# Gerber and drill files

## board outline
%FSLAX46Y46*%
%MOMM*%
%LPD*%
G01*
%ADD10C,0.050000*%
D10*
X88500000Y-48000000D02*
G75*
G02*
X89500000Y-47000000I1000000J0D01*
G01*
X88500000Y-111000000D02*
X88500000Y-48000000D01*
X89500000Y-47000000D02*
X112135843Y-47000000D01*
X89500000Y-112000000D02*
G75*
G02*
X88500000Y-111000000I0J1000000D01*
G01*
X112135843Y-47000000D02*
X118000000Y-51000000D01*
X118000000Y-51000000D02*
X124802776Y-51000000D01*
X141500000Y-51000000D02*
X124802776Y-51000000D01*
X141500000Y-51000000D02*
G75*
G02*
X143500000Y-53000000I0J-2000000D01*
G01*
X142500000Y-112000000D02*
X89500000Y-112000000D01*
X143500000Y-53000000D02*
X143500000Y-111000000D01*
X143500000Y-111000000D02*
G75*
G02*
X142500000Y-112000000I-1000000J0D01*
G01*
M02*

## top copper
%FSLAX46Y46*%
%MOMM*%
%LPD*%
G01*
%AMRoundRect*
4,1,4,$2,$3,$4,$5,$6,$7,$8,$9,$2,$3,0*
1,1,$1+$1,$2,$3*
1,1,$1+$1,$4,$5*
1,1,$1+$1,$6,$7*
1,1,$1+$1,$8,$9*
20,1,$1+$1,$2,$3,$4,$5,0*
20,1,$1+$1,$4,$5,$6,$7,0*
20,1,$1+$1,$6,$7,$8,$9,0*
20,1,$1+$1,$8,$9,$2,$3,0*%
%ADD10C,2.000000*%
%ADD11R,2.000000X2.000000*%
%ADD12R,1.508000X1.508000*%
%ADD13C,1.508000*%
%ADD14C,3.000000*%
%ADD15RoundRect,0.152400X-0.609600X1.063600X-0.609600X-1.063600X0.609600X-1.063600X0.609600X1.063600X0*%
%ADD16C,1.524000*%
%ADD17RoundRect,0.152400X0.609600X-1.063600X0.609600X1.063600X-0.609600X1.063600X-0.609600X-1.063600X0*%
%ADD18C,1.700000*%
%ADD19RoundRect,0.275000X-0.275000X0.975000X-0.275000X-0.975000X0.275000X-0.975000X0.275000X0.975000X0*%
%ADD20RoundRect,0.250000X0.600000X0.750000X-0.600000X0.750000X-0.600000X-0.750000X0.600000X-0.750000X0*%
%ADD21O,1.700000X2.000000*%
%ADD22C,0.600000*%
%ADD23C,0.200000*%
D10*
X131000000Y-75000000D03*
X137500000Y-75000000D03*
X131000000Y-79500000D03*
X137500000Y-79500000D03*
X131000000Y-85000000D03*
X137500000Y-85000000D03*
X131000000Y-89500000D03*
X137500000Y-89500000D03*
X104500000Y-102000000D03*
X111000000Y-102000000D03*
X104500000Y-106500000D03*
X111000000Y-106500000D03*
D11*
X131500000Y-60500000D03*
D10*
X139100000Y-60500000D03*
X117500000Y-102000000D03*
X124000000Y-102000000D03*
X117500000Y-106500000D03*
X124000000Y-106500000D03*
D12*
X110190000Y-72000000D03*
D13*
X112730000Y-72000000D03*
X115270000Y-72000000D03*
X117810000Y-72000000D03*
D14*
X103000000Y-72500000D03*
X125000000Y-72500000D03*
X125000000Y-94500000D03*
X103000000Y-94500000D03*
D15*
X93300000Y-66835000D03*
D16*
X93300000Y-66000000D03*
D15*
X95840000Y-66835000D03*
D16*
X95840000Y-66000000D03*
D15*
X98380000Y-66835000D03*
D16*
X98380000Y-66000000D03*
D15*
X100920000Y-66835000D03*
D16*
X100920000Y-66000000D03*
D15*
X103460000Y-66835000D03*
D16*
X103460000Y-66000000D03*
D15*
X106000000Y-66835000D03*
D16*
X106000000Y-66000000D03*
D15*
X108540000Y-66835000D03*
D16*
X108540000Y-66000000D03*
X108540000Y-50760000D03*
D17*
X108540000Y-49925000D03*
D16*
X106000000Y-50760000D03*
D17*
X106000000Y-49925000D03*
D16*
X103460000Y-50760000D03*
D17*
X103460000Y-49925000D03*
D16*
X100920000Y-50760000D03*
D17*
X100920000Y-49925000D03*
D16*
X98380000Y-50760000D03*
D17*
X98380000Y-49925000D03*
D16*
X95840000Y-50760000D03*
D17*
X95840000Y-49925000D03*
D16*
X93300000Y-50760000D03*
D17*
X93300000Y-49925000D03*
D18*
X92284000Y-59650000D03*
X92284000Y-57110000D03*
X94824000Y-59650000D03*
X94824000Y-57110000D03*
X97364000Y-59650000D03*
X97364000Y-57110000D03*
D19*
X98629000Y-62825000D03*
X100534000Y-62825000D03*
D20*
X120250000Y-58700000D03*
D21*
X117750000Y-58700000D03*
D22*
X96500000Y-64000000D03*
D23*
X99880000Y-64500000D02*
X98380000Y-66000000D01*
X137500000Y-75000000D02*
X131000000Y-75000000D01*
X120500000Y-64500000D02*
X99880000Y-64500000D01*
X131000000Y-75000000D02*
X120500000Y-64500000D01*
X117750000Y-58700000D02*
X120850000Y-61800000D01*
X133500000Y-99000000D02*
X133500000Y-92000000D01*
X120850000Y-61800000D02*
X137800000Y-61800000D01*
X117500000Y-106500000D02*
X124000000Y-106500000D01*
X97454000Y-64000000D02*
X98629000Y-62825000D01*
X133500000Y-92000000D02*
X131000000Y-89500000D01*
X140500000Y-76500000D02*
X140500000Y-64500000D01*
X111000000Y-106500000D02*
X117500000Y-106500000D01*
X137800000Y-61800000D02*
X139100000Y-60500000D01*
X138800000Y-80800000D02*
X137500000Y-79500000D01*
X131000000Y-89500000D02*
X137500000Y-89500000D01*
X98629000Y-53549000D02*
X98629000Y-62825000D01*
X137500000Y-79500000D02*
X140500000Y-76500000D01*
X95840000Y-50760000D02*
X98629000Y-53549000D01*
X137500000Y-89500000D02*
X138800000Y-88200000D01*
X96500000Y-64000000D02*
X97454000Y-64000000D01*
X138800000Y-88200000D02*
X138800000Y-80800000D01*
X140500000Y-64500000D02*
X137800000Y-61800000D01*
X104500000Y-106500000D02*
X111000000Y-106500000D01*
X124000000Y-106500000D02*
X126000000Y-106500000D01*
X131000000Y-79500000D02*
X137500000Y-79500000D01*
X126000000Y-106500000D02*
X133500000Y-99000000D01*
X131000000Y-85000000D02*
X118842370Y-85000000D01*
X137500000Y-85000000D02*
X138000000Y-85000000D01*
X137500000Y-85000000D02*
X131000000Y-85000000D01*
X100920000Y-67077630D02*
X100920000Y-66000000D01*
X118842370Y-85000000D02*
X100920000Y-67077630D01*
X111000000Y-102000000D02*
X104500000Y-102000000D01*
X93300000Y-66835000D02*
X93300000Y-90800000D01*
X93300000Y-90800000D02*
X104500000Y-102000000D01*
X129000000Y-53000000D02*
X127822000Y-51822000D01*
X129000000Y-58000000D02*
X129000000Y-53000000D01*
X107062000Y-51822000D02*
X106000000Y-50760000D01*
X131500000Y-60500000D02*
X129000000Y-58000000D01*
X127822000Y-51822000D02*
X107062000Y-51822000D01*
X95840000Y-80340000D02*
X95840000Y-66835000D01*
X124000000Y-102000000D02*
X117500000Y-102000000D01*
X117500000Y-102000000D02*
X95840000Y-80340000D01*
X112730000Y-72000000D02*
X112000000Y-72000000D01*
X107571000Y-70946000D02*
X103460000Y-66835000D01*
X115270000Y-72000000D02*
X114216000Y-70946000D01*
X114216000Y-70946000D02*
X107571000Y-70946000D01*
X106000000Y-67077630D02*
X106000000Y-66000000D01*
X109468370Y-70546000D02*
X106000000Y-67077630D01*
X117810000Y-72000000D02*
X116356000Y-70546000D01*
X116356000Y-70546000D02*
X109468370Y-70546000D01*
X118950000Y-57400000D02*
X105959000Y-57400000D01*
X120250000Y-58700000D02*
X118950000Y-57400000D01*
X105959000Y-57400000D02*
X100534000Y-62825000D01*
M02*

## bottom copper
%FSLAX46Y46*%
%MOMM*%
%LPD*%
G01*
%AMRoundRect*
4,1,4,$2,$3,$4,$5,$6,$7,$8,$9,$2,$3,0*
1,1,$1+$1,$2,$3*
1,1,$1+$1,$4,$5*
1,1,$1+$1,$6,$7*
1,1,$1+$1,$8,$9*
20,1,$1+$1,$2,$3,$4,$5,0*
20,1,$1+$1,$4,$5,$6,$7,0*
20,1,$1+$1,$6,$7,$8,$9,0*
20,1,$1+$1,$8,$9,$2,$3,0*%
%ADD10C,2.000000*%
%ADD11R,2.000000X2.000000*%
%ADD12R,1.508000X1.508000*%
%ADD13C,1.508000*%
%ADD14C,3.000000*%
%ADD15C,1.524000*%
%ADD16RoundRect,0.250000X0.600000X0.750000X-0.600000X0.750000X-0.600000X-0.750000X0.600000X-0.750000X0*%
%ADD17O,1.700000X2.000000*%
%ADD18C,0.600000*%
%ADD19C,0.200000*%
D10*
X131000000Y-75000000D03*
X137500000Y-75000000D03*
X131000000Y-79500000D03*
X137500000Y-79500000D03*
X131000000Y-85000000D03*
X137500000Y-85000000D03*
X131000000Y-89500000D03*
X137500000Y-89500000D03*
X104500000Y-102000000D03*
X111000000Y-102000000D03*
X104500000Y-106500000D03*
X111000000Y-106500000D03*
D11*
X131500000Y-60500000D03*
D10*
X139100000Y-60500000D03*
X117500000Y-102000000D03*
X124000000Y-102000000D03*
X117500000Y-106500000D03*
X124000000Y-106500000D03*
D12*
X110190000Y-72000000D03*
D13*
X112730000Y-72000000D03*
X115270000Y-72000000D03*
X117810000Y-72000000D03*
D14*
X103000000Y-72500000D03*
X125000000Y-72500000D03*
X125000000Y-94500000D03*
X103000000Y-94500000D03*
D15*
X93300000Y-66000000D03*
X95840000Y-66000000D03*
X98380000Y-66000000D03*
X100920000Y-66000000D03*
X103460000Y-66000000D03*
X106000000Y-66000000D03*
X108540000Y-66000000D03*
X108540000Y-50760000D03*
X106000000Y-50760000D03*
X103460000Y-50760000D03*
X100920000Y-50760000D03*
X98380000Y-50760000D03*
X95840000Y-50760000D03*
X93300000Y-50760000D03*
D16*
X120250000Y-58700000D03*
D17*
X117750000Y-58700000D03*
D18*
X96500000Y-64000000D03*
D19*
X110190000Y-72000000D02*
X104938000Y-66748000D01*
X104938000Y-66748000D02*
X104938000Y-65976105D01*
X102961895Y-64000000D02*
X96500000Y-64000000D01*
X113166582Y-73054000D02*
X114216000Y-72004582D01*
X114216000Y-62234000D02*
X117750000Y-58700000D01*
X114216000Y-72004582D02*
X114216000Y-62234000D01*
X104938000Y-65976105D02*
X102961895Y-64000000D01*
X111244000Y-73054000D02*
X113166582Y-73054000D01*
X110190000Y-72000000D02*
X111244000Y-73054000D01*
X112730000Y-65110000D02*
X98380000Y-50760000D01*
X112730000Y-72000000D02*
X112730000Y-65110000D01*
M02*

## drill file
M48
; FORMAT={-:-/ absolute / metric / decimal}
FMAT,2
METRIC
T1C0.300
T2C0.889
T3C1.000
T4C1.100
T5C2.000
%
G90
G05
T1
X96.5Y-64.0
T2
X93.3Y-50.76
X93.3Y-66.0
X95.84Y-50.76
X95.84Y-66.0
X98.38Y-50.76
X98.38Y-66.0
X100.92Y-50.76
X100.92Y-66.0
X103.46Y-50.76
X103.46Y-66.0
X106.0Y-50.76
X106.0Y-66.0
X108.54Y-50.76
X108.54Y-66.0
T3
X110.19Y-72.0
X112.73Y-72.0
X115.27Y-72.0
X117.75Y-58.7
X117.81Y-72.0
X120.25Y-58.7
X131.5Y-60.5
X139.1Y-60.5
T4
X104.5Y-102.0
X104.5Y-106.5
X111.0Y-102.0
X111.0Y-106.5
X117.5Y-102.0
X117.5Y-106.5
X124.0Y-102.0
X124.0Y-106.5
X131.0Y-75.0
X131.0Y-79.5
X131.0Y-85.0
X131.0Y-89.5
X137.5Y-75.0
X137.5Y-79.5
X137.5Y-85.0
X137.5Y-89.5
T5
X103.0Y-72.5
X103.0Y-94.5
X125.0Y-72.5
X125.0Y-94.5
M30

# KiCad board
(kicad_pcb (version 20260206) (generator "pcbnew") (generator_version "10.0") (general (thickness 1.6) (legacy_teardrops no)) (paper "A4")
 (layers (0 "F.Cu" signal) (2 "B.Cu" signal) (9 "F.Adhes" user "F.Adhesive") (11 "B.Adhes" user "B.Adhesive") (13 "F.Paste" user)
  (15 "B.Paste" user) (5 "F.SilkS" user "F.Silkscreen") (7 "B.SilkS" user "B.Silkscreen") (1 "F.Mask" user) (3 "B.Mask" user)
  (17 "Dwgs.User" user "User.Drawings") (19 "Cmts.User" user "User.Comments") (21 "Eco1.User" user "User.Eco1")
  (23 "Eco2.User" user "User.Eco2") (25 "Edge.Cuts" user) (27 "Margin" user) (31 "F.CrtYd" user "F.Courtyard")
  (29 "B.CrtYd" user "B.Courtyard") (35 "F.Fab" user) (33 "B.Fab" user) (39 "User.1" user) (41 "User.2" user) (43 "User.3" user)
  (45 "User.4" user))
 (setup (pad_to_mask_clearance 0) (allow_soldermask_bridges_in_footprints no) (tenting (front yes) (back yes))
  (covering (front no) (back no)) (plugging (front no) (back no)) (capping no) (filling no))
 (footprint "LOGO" (layer "F.Cu") (at 95 102)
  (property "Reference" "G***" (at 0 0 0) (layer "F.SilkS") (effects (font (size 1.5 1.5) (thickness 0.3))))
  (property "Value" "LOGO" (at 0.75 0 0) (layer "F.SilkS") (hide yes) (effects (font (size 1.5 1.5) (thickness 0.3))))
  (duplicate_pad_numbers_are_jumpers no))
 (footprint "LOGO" (layer "F.Cu") (at 124.5 55.5)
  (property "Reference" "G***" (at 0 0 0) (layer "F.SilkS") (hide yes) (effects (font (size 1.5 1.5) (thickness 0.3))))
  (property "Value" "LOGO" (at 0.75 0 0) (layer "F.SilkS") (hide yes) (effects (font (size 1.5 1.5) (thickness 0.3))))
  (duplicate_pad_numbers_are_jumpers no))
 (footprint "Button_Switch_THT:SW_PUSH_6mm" (layer "F.Cu") (at 131 75)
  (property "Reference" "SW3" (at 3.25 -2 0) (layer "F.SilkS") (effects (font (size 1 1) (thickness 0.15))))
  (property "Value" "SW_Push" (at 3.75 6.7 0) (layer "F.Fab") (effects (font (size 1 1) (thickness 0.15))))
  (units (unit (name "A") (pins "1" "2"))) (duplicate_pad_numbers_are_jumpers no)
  (pad "1" thru_hole circle (at 0 0 90) (size 2 2) (drill 1.1) (layers "*.Cu" "*.Mask") (remove_unused_layers no) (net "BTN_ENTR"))
  (pad "1" thru_hole circle (at 6.5 0 90) (size 2 2) (drill 1.1) (layers "*.Cu" "*.Mask") (remove_unused_layers no) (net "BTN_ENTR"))
  (pad "2" thru_hole circle (at 0 4.5 90) (size 2 2) (drill 1.1) (layers "*.Cu" "*.Mask") (remove_unused_layers no) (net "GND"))
  (pad "2" thru_hole circle (at 6.5 4.5 90) (size 2 2) (drill 1.1) (layers "*.Cu" "*.Mask") (remove_unused_layers no) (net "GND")))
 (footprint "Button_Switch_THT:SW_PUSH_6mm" (layer "F.Cu") (at 131 85)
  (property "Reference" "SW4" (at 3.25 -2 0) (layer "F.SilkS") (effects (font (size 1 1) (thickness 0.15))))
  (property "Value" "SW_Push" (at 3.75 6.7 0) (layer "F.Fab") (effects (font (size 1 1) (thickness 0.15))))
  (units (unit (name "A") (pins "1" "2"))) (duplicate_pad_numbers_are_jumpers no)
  (pad "1" thru_hole circle (at 0 0 90) (size 2 2) (drill 1.1) (layers "*.Cu" "*.Mask") (remove_unused_layers no) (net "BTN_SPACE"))
  (pad "1" thru_hole circle (at 6.5 0 90) (size 2 2) (drill 1.1) (layers "*.Cu" "*.Mask") (remove_unused_layers no) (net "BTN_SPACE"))
  (pad "2" thru_hole circle (at 0 4.5 90) (size 2 2) (drill 1.1) (layers "*.Cu" "*.Mask") (remove_unused_layers no) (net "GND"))
  (pad "2" thru_hole circle (at 6.5 4.5 90) (size 2 2) (drill 1.1) (layers "*.Cu" "*.Mask") (remove_unused_layers no) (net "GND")))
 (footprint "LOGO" (layer "F.Cu") (at 123 55.5)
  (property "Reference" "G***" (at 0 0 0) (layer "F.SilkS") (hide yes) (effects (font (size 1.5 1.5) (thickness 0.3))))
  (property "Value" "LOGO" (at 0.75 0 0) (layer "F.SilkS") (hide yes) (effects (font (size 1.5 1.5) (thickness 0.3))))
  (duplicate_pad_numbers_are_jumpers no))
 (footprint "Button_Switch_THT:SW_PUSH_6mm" (layer "F.Cu") (at 104.5 102)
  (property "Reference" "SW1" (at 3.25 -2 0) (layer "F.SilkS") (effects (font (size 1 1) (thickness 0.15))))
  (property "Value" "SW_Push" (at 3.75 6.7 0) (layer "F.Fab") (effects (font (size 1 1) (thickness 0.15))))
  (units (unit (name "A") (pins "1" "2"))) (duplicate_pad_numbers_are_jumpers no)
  (pad "1" thru_hole circle (at 0 0 90) (size 2 2) (drill 1.1) (layers "*.Cu" "*.Mask") (remove_unused_layers no) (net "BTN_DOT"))
  (pad "1" thru_hole circle (at 6.5 0 90) (size 2 2) (drill 1.1) (layers "*.Cu" "*.Mask") (remove_unused_layers no) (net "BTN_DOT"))
  (pad "2" thru_hole circle (at 0 4.5 90) (size 2 2) (drill 1.1) (layers "*.Cu" "*.Mask") (remove_unused_layers no) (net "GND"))
  (pad "2" thru_hole circle (at 6.5 4.5 90) (size 2 2) (drill 1.1) (layers "*.Cu" "*.Mask") (remove_unused_layers no) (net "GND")))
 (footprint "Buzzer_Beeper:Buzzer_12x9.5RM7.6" (layer "F.Cu") (at 131.5 60.5)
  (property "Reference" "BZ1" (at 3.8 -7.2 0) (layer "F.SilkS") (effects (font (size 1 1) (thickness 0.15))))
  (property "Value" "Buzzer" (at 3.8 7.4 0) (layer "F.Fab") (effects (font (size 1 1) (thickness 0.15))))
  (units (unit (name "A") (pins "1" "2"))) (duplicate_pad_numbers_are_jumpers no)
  (pad "1" thru_hole rect (at 0 0) (size 2 2) (drill 1) (layers "*.Cu" "*.Mask") (remove_unused_layers no) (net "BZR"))
  (pad "2" thru_hole circle (at 7.6 0) (size 2 2) (drill 1) (layers "*.Cu" "*.Mask") (remove_unused_layers no) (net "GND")))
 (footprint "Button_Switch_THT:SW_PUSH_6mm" (layer "F.Cu") (at 117.5 102)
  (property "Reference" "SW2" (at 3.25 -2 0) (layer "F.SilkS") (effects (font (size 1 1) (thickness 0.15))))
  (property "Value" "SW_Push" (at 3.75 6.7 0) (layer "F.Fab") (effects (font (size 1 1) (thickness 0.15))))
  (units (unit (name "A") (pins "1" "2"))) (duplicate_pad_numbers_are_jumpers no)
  (pad "1" thru_hole circle (at 0 0 90) (size 2 2) (drill 1.1) (layers "*.Cu" "*.Mask") (remove_unused_layers no) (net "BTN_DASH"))
  (pad "1" thru_hole circle (at 6.5 0 90) (size 2 2) (drill 1.1) (layers "*.Cu" "*.Mask") (remove_unused_layers no) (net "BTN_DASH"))
  (pad "2" thru_hole circle (at 0 4.5 90) (size 2 2) (drill 1.1) (layers "*.Cu" "*.Mask") (remove_unused_layers no) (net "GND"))
  (pad "2" thru_hole circle (at 6.5 4.5 90) (size 2 2) (drill 1.1) (layers "*.Cu" "*.Mask") (remove_unused_layers no) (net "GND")))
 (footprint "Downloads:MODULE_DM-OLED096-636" (layer "F.Cu") (at 114 83.5)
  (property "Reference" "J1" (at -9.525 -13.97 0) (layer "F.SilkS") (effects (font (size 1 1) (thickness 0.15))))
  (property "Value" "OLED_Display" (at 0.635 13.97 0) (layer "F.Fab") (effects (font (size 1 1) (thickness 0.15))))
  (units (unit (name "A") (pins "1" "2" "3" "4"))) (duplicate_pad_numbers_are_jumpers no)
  (pad "1" thru_hole rect (at -3.81 -11.5) (size 1.508 1.508) (drill 1) (layers "*.Cu" "*.Mask") (remove_unused_layers no) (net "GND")
   (solder_mask_margin 0.102))
  (pad "2" thru_hole circle (at -1.27 -11.5) (size 1.508 1.508) (drill 1) (layers "*.Cu" "*.Mask") (remove_unused_layers no) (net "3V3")
   (solder_mask_margin 0.102))
  (pad "3" thru_hole circle (at 1.27 -11.5) (size 1.508 1.508) (drill 1) (layers "*.Cu" "*.Mask") (remove_unused_layers no) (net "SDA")
   (solder_mask_margin 0.102))
  (pad "4" thru_hole circle (at 3.81 -11.5) (size 1.508 1.508) (drill 1) (layers "*.Cu" "*.Mask") (remove_unused_layers no) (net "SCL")
   (solder_mask_margin 0.102))
  (pad "S1" thru_hole circle (at -11 -11) (size 3 3) (drill 2) (layers "*.Cu" "*.Mask") (remove_unused_layers no) (solder_mask_margin 0.102))
  (pad "S2" thru_hole circle (at 11 -11) (size 3 3) (drill 2) (layers "*.Cu" "*.Mask") (remove_unused_layers no) (solder_mask_margin 0.102))
  (pad "S3" thru_hole circle (at 11 11) (size 3 3) (drill 2) (layers "*.Cu" "*.Mask") (remove_unused_layers no) (solder_mask_margin 0.102))
  (pad "S4" thru_hole circle (at -11 11) (size 3 3) (drill 2) (layers "*.Cu" "*.Mask") (remove_unused_layers no) (solder_mask_margin 0.102)))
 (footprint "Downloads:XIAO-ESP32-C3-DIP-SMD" (layer "F.Cu") (at 100.92 58.38 180)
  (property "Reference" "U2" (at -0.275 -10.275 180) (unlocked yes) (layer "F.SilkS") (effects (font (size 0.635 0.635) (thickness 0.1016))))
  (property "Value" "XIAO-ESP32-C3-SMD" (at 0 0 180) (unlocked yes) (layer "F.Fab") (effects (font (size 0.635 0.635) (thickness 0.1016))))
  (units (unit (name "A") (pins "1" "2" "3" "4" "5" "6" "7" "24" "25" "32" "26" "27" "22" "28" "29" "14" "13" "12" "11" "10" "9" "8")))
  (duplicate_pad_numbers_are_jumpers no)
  (pad "1" smd roundrect (at 7.62 -8.455 270) (size 2.432 1.524) (layers "F.Cu" "F.Mask") (roundrect_rratio 0.1) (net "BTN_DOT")
   (thermal_bridge_angle 45))
  (pad "1" thru_hole circle (at 7.62 -7.62 270) (size 1.524 1.524) (drill 0.889) (layers "*.Cu" "*.Mask") (remove_unused_layers no)
   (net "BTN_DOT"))
  (pad "2" smd roundrect (at 5.08 -8.455 270) (size 2.432 1.524) (layers "F.Cu" "F.Mask") (roundrect_rratio 0.1) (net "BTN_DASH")
   (thermal_bridge_angle 45))
  (pad "2" thru_hole circle (at 5.08 -7.62 270) (size 1.524 1.524) (drill 0.889) (layers "*.Cu" "*.Mask") (remove_unused_layers no)
   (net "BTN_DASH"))
  (pad "3" smd roundrect (at 2.54 -8.455 270) (size 2.432 1.524) (layers "F.Cu" "F.Mask") (roundrect_rratio 0.1) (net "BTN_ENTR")
   (thermal_bridge_angle 45))
  (pad "3" thru_hole circle (at 2.54 -7.62 270) (size 1.524 1.524) (drill 0.889) (layers "*.Cu" "*.Mask") (remove_unused_layers no)
   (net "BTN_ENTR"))
  (pad "4" smd roundrect (at 0 -8.455 270) (size 2.432 1.524) (layers "F.Cu" "F.Mask") (roundrect_rratio 0.1) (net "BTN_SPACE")
   (thermal_bridge_angle 45))
  (pad "4" thru_hole circle (at 0 -7.62 270) (size 1.524 1.524) (drill 0.889) (layers "*.Cu" "*.Mask") (remove_unused_layers no)
   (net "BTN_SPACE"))
  (pad "5" smd roundrect (at -2.54 -8.455 270) (size 2.432 1.524) (layers "F.Cu" "F.Mask") (roundrect_rratio 0.1) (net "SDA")
   (thermal_bridge_angle 45))
  (pad "5" thru_hole circle (at -2.54 -7.62 270) (size 1.524 1.524) (drill 0.889) (layers "*.Cu" "*.Mask") (remove_unused_layers no)
   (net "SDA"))
  (pad "6" smd roundrect (at -5.08 -8.455 270) (size 2.432 1.524) (layers "F.Cu" "F.Mask") (roundrect_rratio 0.1) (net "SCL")
   (thermal_bridge_angle 45))
  (pad "6" thru_hole circle (at -5.08 -7.62 270) (size 1.524 1.524) (drill 0.889) (layers "*.Cu" "*.Mask") (remove_unused_layers no)
   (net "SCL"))
  (pad "7" smd roundrect (at -7.62 -8.455 270) (size 2.432 1.524) (layers "F.Cu" "F.Mask") (roundrect_rratio 0.1)
   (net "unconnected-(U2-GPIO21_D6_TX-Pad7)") (thermal_bridge_angle 45))
  (pad "7" thru_hole circle (at -7.62 -7.62 270) (size 1.524 1.524) (drill 0.889) (layers "*.Cu" "*.Mask") (remove_unused_layers no)
   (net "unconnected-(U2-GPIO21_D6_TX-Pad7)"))
  (pad "8" thru_hole circle (at -7.62 7.62 90) (size 1.524 1.524) (drill 0.889) (layers "*.Cu" "*.Mask") (remove_unused_layers no)
   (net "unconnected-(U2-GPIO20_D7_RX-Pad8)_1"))
  (pad "8" smd roundrect (at -7.62 8.455 90) (size 2.432 1.524) (layers "F.Cu" "F.Mask") (roundrect_rratio 0.1)
   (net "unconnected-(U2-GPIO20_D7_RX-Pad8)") (thermal_bridge_angle 45))
  (pad "9" thru_hole circle (at -5.08 7.62 90) (size 1.524 1.524) (drill 0.889) (layers "*.Cu" "*.Mask") (remove_unused_layers no)
   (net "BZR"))
  (pad "9" smd roundrect (at -5.08 8.455 90) (size 2.432 1.524) (layers "F.Cu" "F.Mask") (roundrect_rratio 0.1) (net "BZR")
   (thermal_bridge_angle 45))
  (pad "10" thru_hole circle (at -2.54 7.62 90) (size 1.524 1.524) (drill 0.889) (layers "*.Cu" "*.Mask") (remove_unused_layers no)
   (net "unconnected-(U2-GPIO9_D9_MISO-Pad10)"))
  (pad "10" smd roundrect (at -2.54 8.455 90) (size 2.432 1.524) (layers "F.Cu" "F.Mask") (roundrect_rratio 0.1)
   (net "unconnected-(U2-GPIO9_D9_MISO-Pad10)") (thermal_bridge_angle 45))
  (pad "11" thru_hole circle (at 0 7.62 90) (size 1.524 1.524) (drill 0.889) (layers "*.Cu" "*.Mask") (remove_unused_layers no)
   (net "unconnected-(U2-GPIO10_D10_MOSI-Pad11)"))
  (pad "11" smd roundrect (at 0 8.455 90) (size 2.432 1.524) (layers "F.Cu" "F.Mask") (roundrect_rratio 0.1)
   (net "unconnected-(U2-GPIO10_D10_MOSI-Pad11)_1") (thermal_bridge_angle 45))
  (pad "12" thru_hole circle (at 2.54 7.62 90) (size 1.524 1.524) (drill 0.889) (layers "*.Cu" "*.Mask") (remove_unused_layers no)
   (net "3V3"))
  (pad "12" smd roundrect (at 2.54 8.455 90) (size 2.432 1.524) (layers "F.Cu" "F.Mask") (roundrect_rratio 0.1) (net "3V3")
   (thermal_bridge_angle 45))
  (pad "13" thru_hole circle (at 5.08 7.62 90) (size 1.524 1.524) (drill 0.889) (layers "*.Cu" "*.Mask") (remove_unused_layers no)
   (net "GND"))
  (pad "13" smd roundrect (at 5.08 8.455 90) (size 2.432 1.524) (layers "F.Cu" "F.Mask") (roundrect_rratio 0.1) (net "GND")
   (thermal_bridge_angle 45))
  (pad "14" thru_hole circle (at 7.62 7.62 90) (size 1.524 1.524) (drill 0.889) (layers "*.Cu" "*.Mask") (remove_unused_layers no)
   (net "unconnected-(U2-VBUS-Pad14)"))
  (pad "14" smd roundrect (at 7.62 8.455 90) (size 2.432 1.524) (layers "F.Cu" "F.Mask") (roundrect_rratio 0.1)
   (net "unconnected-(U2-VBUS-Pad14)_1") (thermal_bridge_angle 45))
  (pad "15" smd circle (at 8.636 -1.27 90) (size 1.7 1.7) (layers "F.Cu" "F.Mask" "F.Paste"))
  (pad "16" smd circle (at 8.636 1.27 90) (size 1.7 1.7) (layers "F.Cu" "F.Mask" "F.Paste"))
  (pad "17" smd circle (at 6.096 -1.27 90) (size 1.7 1.7) (layers "F.Cu" "F.Mask" "F.Paste"))
  (pad "18" smd circle (at 6.096 1.27 90) (size 1.7 1.7) (layers "F.Cu" "F.Mask" "F.Paste"))
  (pad "19" smd circle (at 3.556 -1.27 90) (size 1.7 1.7) (layers "F.Cu" "F.Mask" "F.Paste"))
  (pad "20" smd circle (at 3.556 1.27 90) (size 1.7 1.7) (layers "F.Cu" "F.Mask" "F.Paste"))
  (pad "22" smd roundrect (at 2.291 -4.445 270) (size 2.5 1.1) (layers "F.Cu" "F.Mask" "F.Paste") (roundrect_rratio 0.25) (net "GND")
   (thermal_bridge_angle 45))
  (pad "32" smd roundrect (at 0.386 -4.445 270) (size 2.5 1.1) (layers "F.Cu" "F.Mask" "F.Paste") (roundrect_rratio 0.25) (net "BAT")
   (thermal_bridge_angle 45)))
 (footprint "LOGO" (layer "F.Cu") (at 121.5 55.5)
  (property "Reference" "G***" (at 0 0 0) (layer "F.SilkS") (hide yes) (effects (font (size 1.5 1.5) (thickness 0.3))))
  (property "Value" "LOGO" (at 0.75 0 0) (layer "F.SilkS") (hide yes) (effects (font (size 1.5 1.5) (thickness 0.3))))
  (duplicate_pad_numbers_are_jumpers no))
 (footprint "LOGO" (layer "B.Cu") (at 113.293261 85.085018 180)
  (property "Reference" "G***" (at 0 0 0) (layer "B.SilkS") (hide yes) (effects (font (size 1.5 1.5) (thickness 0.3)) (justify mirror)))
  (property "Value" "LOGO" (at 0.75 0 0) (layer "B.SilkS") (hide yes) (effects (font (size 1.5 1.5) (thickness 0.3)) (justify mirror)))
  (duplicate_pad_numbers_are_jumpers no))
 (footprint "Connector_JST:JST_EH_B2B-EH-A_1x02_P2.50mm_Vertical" (layer "B.Cu") (at 120.25 58.7 180)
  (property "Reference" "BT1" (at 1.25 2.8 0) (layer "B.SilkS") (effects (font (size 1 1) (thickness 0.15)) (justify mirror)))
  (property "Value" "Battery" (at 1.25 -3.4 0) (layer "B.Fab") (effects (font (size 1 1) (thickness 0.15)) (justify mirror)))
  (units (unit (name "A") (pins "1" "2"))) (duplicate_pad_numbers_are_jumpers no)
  (pad "1" thru_hole roundrect (at 0 0 180) (size 1.7 2) (drill 1) (layers "*.Cu" "*.Mask") (remove_unused_layers no)
   (roundrect_rratio 0.147059) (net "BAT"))
  (pad "2" thru_hole oval (at 2.5 0 180) (size 1.7 2) (drill 1) (layers "*.Cu" "*.Mask") (remove_unused_layers no) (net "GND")))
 (gr_arc (start 88.5 48) (mid 88.792893 47.292893) (end 89.5 47) (stroke (width 0.05) (type default)) (layer "Edge.Cuts"))
 (gr_line (start 88.5 111) (end 88.5 48) (stroke (width 0.05) (type default)) (layer "Edge.Cuts"))
 (gr_line (start 89.5 47) (end 112.135843 47) (stroke (width 0.05) (type default)) (layer "Edge.Cuts"))
 (gr_arc (start 89.5 112) (mid 88.792893 111.707107) (end 88.5 111) (stroke (width 0.05) (type default)) (layer "Edge.Cuts"))
 (gr_line (start 112.135843 47) (end 118 51) (stroke (width 0.05) (type default)) (layer "Edge.Cuts"))
 (gr_line (start 118 51) (end 124.802776 51) (stroke (width 0.05) (type default)) (layer "Edge.Cuts"))
 (gr_line (start 141.5 51) (end 124.802776 51) (stroke (width 0.05) (type default)) (layer "Edge.Cuts"))
 (gr_arc (start 141.5 51) (mid 142.914214 51.585786) (end 143.5 53) (stroke (width 0.05) (type default)) (layer "Edge.Cuts"))
 (gr_line (start 142.5 112) (end 89.5 112) (stroke (width 0.05) (type default)) (layer "Edge.Cuts"))
 (gr_line (start 143.5 53) (end 143.5 111) (stroke (width 0.05) (type default)) (layer "Edge.Cuts"))
 (gr_arc (start 143.5 111) (mid 143.207107 111.707107) (end 142.5 112) (stroke (width 0.05) (type default)) (layer "Edge.Cuts"))
 (segment (start 99.88 64.5) (end 98.38 66) (width 0.2) (layer "F.Cu") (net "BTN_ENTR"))
 (segment (start 137.5 75) (end 131 75) (width 0.2) (layer "F.Cu") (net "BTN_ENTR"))
 (segment (start 120.5 64.5) (end 99.88 64.5) (width 0.2) (layer "F.Cu") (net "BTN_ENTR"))
 (segment (start 131 75) (end 120.5 64.5) (width 0.2) (layer "F.Cu") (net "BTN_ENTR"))
 (segment (start 117.75 58.7) (end 120.85 61.8) (width 0.2) (layer "F.Cu") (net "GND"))
 (segment (start 133.5 99) (end 133.5 92) (width 0.2) (layer "F.Cu") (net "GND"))
 (segment (start 120.85 61.8) (end 137.8 61.8) (width 0.2) (layer "F.Cu") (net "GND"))
 (segment (start 117.5 106.5) (end 124 106.5) (width 0.2) (layer "F.Cu") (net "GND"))
 (segment (start 97.454 64) (end 98.629 62.825) (width 0.2) (layer "F.Cu") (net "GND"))
 (segment (start 133.5 92) (end 131 89.5) (width 0.2) (layer "F.Cu") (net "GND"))
 (segment (start 140.5 76.5) (end 140.5 64.5) (width 0.2) (layer "F.Cu") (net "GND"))
 (segment (start 111 106.5) (end 117.5 106.5) (width 0.2) (layer "F.Cu") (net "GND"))
 (segment (start 137.8 61.8) (end 139.1 60.5) (width 0.2) (layer "F.Cu") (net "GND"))
 (segment (start 138.8 80.8) (end 137.5 79.5) (width 0.2) (layer "F.Cu") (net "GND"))
 (segment (start 131 89.5) (end 137.5 89.5) (width 0.2) (layer "F.Cu") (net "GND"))
 (segment (start 98.629 53.549) (end 98.629 62.825) (width 0.2) (layer "F.Cu") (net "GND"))
 (segment (start 137.5 79.5) (end 140.5 76.5) (width 0.2) (layer "F.Cu") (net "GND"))
 (segment (start 95.84 50.76) (end 98.629 53.549) (width 0.2) (layer "F.Cu") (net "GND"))
 (segment (start 137.5 89.5) (end 138.8 88.2) (width 0.2) (layer "F.Cu") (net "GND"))
 (segment (start 96.5 64) (end 97.454 64) (width 0.2) (layer "F.Cu") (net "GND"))
 (segment (start 138.8 88.2) (end 138.8 80.8) (width 0.2) (layer "F.Cu") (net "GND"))
 (segment (start 140.5 64.5) (end 137.8 61.8) (width 0.2) (layer "F.Cu") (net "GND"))
 (segment (start 104.5 106.5) (end 111 106.5) (width 0.2) (layer "F.Cu") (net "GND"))
 (segment (start 124 106.5) (end 126 106.5) (width 0.2) (layer "F.Cu") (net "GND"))
 (segment (start 131 79.5) (end 137.5 79.5) (width 0.2) (layer "F.Cu") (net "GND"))
 (segment (start 126 106.5) (end 133.5 99) (width 0.2) (layer "F.Cu") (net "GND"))
 (via (at 96.5 64) (size 0.6) (drill 0.3) (layers "F.Cu" "B.Cu") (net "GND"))
 (segment (start 110.19 72) (end 104.938 66.748) (width 0.2) (layer "B.Cu") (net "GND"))
 (segment (start 104.938 66.748) (end 104.938 65.976105) (width 0.2) (layer "B.Cu") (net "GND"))
 (segment (start 102.961895 64) (end 96.5 64) (width 0.2) (layer "B.Cu") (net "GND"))
 (segment (start 113.166582 73.054) (end 114.216 72.004582) (width 0.2) (layer "B.Cu") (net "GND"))
 (segment (start 114.216 62.234) (end 117.75 58.7) (width 0.2) (layer "B.Cu") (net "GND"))
 (segment (start 114.216 72.004582) (end 114.216 62.234) (width 0.2) (layer "B.Cu") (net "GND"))
 (segment (start 104.938 65.976105) (end 102.961895 64) (width 0.2) (layer "B.Cu") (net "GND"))
 (segment (start 111.244 73.054) (end 113.166582 73.054) (width 0.2) (layer "B.Cu") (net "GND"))
 (segment (start 110.19 72) (end 111.244 73.054) (width 0.2) (layer "B.Cu") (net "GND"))
 (segment (start 131 85) (end 118.84237 85) (width 0.2) (layer "F.Cu") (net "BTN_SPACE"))
 (segment (start 137.5 85) (end 138 85) (width 0.2) (layer "F.Cu") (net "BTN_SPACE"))
 (segment (start 137.5 85) (end 131 85) (width 0.2) (layer "F.Cu") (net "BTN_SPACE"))
 (segment (start 100.92 67.07763) (end 100.92 66) (width 0.2) (layer "F.Cu") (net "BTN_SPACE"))
 (segment (start 118.84237 85) (end 100.92 67.07763) (width 0.2) (layer "F.Cu") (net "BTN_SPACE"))
 (segment (start 111 102) (end 104.5 102) (width 0.2) (layer "F.Cu") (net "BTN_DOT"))
 (segment (start 93.3 66.835) (end 93.3 90.8) (width 0.2) (layer "F.Cu") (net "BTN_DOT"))
 (segment (start 93.3 90.8) (end 104.5 102) (width 0.2) (layer "F.Cu") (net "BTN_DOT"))
 (segment (start 129 53) (end 127.822 51.822) (width 0.2) (layer "F.Cu") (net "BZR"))
 (segment (start 129 58) (end 129 53) (width 0.2) (layer "F.Cu") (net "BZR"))
 (segment (start 107.062 51.822) (end 106 50.76) (width 0.2) (layer "F.Cu") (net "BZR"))
 (segment (start 131.5 60.5) (end 129 58) (width 0.2) (layer "F.Cu") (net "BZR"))
 (segment (start 127.822 51.822) (end 107.062 51.822) (width 0.2) (layer "F.Cu") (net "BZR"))
 (segment (start 95.84 80.34) (end 95.84 66.835) (width 0.2) (layer "F.Cu") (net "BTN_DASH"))
 (segment (start 124 102) (end 117.5 102) (width 0.2) (layer "F.Cu") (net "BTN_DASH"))
 (segment (start 117.5 102) (end 95.84 80.34) (width 0.2) (layer "F.Cu") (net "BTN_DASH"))
 (segment (start 112.73 72) (end 112 72) (width 0.2) (layer "F.Cu") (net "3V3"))
 (segment (start 112.73 65.11) (end 98.38 50.76) (width 0.2) (layer "B.Cu") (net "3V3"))
 (segment (start 112.73 72) (end 112.73 65.11) (width 0.2) (layer "B.Cu") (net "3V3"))
 (segment (start 107.571 70.946) (end 103.46 66.835) (width 0.2) (layer "F.Cu") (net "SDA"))
 (segment (start 115.27 72) (end 114.216 70.946) (width 0.2) (layer "F.Cu") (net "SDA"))
 (segment (start 114.216 70.946) (end 107.571 70.946) (width 0.2) (layer "F.Cu") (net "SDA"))
 (segment (start 106 67.07763) (end 106 66) (width 0.2) (layer "F.Cu") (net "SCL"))
 (segment (start 109.46837 70.546) (end 106 67.07763) (width 0.2) (layer "F.Cu") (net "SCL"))
 (segment (start 117.81 72) (end 116.356 70.546) (width 0.2) (layer "F.Cu") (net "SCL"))
 (segment (start 116.356 70.546) (end 109.46837 70.546) (width 0.2) (layer "F.Cu") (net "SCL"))
 (segment (start 118.95 57.4) (end 105.959 57.4) (width 0.2) (layer "F.Cu") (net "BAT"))
 (segment (start 120.25 58.7) (end 118.95 57.4) (width 0.2) (layer "F.Cu") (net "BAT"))
 (segment (start 105.959 57.4) (end 100.534 62.825) (width 0.2) (layer "F.Cu") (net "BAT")))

